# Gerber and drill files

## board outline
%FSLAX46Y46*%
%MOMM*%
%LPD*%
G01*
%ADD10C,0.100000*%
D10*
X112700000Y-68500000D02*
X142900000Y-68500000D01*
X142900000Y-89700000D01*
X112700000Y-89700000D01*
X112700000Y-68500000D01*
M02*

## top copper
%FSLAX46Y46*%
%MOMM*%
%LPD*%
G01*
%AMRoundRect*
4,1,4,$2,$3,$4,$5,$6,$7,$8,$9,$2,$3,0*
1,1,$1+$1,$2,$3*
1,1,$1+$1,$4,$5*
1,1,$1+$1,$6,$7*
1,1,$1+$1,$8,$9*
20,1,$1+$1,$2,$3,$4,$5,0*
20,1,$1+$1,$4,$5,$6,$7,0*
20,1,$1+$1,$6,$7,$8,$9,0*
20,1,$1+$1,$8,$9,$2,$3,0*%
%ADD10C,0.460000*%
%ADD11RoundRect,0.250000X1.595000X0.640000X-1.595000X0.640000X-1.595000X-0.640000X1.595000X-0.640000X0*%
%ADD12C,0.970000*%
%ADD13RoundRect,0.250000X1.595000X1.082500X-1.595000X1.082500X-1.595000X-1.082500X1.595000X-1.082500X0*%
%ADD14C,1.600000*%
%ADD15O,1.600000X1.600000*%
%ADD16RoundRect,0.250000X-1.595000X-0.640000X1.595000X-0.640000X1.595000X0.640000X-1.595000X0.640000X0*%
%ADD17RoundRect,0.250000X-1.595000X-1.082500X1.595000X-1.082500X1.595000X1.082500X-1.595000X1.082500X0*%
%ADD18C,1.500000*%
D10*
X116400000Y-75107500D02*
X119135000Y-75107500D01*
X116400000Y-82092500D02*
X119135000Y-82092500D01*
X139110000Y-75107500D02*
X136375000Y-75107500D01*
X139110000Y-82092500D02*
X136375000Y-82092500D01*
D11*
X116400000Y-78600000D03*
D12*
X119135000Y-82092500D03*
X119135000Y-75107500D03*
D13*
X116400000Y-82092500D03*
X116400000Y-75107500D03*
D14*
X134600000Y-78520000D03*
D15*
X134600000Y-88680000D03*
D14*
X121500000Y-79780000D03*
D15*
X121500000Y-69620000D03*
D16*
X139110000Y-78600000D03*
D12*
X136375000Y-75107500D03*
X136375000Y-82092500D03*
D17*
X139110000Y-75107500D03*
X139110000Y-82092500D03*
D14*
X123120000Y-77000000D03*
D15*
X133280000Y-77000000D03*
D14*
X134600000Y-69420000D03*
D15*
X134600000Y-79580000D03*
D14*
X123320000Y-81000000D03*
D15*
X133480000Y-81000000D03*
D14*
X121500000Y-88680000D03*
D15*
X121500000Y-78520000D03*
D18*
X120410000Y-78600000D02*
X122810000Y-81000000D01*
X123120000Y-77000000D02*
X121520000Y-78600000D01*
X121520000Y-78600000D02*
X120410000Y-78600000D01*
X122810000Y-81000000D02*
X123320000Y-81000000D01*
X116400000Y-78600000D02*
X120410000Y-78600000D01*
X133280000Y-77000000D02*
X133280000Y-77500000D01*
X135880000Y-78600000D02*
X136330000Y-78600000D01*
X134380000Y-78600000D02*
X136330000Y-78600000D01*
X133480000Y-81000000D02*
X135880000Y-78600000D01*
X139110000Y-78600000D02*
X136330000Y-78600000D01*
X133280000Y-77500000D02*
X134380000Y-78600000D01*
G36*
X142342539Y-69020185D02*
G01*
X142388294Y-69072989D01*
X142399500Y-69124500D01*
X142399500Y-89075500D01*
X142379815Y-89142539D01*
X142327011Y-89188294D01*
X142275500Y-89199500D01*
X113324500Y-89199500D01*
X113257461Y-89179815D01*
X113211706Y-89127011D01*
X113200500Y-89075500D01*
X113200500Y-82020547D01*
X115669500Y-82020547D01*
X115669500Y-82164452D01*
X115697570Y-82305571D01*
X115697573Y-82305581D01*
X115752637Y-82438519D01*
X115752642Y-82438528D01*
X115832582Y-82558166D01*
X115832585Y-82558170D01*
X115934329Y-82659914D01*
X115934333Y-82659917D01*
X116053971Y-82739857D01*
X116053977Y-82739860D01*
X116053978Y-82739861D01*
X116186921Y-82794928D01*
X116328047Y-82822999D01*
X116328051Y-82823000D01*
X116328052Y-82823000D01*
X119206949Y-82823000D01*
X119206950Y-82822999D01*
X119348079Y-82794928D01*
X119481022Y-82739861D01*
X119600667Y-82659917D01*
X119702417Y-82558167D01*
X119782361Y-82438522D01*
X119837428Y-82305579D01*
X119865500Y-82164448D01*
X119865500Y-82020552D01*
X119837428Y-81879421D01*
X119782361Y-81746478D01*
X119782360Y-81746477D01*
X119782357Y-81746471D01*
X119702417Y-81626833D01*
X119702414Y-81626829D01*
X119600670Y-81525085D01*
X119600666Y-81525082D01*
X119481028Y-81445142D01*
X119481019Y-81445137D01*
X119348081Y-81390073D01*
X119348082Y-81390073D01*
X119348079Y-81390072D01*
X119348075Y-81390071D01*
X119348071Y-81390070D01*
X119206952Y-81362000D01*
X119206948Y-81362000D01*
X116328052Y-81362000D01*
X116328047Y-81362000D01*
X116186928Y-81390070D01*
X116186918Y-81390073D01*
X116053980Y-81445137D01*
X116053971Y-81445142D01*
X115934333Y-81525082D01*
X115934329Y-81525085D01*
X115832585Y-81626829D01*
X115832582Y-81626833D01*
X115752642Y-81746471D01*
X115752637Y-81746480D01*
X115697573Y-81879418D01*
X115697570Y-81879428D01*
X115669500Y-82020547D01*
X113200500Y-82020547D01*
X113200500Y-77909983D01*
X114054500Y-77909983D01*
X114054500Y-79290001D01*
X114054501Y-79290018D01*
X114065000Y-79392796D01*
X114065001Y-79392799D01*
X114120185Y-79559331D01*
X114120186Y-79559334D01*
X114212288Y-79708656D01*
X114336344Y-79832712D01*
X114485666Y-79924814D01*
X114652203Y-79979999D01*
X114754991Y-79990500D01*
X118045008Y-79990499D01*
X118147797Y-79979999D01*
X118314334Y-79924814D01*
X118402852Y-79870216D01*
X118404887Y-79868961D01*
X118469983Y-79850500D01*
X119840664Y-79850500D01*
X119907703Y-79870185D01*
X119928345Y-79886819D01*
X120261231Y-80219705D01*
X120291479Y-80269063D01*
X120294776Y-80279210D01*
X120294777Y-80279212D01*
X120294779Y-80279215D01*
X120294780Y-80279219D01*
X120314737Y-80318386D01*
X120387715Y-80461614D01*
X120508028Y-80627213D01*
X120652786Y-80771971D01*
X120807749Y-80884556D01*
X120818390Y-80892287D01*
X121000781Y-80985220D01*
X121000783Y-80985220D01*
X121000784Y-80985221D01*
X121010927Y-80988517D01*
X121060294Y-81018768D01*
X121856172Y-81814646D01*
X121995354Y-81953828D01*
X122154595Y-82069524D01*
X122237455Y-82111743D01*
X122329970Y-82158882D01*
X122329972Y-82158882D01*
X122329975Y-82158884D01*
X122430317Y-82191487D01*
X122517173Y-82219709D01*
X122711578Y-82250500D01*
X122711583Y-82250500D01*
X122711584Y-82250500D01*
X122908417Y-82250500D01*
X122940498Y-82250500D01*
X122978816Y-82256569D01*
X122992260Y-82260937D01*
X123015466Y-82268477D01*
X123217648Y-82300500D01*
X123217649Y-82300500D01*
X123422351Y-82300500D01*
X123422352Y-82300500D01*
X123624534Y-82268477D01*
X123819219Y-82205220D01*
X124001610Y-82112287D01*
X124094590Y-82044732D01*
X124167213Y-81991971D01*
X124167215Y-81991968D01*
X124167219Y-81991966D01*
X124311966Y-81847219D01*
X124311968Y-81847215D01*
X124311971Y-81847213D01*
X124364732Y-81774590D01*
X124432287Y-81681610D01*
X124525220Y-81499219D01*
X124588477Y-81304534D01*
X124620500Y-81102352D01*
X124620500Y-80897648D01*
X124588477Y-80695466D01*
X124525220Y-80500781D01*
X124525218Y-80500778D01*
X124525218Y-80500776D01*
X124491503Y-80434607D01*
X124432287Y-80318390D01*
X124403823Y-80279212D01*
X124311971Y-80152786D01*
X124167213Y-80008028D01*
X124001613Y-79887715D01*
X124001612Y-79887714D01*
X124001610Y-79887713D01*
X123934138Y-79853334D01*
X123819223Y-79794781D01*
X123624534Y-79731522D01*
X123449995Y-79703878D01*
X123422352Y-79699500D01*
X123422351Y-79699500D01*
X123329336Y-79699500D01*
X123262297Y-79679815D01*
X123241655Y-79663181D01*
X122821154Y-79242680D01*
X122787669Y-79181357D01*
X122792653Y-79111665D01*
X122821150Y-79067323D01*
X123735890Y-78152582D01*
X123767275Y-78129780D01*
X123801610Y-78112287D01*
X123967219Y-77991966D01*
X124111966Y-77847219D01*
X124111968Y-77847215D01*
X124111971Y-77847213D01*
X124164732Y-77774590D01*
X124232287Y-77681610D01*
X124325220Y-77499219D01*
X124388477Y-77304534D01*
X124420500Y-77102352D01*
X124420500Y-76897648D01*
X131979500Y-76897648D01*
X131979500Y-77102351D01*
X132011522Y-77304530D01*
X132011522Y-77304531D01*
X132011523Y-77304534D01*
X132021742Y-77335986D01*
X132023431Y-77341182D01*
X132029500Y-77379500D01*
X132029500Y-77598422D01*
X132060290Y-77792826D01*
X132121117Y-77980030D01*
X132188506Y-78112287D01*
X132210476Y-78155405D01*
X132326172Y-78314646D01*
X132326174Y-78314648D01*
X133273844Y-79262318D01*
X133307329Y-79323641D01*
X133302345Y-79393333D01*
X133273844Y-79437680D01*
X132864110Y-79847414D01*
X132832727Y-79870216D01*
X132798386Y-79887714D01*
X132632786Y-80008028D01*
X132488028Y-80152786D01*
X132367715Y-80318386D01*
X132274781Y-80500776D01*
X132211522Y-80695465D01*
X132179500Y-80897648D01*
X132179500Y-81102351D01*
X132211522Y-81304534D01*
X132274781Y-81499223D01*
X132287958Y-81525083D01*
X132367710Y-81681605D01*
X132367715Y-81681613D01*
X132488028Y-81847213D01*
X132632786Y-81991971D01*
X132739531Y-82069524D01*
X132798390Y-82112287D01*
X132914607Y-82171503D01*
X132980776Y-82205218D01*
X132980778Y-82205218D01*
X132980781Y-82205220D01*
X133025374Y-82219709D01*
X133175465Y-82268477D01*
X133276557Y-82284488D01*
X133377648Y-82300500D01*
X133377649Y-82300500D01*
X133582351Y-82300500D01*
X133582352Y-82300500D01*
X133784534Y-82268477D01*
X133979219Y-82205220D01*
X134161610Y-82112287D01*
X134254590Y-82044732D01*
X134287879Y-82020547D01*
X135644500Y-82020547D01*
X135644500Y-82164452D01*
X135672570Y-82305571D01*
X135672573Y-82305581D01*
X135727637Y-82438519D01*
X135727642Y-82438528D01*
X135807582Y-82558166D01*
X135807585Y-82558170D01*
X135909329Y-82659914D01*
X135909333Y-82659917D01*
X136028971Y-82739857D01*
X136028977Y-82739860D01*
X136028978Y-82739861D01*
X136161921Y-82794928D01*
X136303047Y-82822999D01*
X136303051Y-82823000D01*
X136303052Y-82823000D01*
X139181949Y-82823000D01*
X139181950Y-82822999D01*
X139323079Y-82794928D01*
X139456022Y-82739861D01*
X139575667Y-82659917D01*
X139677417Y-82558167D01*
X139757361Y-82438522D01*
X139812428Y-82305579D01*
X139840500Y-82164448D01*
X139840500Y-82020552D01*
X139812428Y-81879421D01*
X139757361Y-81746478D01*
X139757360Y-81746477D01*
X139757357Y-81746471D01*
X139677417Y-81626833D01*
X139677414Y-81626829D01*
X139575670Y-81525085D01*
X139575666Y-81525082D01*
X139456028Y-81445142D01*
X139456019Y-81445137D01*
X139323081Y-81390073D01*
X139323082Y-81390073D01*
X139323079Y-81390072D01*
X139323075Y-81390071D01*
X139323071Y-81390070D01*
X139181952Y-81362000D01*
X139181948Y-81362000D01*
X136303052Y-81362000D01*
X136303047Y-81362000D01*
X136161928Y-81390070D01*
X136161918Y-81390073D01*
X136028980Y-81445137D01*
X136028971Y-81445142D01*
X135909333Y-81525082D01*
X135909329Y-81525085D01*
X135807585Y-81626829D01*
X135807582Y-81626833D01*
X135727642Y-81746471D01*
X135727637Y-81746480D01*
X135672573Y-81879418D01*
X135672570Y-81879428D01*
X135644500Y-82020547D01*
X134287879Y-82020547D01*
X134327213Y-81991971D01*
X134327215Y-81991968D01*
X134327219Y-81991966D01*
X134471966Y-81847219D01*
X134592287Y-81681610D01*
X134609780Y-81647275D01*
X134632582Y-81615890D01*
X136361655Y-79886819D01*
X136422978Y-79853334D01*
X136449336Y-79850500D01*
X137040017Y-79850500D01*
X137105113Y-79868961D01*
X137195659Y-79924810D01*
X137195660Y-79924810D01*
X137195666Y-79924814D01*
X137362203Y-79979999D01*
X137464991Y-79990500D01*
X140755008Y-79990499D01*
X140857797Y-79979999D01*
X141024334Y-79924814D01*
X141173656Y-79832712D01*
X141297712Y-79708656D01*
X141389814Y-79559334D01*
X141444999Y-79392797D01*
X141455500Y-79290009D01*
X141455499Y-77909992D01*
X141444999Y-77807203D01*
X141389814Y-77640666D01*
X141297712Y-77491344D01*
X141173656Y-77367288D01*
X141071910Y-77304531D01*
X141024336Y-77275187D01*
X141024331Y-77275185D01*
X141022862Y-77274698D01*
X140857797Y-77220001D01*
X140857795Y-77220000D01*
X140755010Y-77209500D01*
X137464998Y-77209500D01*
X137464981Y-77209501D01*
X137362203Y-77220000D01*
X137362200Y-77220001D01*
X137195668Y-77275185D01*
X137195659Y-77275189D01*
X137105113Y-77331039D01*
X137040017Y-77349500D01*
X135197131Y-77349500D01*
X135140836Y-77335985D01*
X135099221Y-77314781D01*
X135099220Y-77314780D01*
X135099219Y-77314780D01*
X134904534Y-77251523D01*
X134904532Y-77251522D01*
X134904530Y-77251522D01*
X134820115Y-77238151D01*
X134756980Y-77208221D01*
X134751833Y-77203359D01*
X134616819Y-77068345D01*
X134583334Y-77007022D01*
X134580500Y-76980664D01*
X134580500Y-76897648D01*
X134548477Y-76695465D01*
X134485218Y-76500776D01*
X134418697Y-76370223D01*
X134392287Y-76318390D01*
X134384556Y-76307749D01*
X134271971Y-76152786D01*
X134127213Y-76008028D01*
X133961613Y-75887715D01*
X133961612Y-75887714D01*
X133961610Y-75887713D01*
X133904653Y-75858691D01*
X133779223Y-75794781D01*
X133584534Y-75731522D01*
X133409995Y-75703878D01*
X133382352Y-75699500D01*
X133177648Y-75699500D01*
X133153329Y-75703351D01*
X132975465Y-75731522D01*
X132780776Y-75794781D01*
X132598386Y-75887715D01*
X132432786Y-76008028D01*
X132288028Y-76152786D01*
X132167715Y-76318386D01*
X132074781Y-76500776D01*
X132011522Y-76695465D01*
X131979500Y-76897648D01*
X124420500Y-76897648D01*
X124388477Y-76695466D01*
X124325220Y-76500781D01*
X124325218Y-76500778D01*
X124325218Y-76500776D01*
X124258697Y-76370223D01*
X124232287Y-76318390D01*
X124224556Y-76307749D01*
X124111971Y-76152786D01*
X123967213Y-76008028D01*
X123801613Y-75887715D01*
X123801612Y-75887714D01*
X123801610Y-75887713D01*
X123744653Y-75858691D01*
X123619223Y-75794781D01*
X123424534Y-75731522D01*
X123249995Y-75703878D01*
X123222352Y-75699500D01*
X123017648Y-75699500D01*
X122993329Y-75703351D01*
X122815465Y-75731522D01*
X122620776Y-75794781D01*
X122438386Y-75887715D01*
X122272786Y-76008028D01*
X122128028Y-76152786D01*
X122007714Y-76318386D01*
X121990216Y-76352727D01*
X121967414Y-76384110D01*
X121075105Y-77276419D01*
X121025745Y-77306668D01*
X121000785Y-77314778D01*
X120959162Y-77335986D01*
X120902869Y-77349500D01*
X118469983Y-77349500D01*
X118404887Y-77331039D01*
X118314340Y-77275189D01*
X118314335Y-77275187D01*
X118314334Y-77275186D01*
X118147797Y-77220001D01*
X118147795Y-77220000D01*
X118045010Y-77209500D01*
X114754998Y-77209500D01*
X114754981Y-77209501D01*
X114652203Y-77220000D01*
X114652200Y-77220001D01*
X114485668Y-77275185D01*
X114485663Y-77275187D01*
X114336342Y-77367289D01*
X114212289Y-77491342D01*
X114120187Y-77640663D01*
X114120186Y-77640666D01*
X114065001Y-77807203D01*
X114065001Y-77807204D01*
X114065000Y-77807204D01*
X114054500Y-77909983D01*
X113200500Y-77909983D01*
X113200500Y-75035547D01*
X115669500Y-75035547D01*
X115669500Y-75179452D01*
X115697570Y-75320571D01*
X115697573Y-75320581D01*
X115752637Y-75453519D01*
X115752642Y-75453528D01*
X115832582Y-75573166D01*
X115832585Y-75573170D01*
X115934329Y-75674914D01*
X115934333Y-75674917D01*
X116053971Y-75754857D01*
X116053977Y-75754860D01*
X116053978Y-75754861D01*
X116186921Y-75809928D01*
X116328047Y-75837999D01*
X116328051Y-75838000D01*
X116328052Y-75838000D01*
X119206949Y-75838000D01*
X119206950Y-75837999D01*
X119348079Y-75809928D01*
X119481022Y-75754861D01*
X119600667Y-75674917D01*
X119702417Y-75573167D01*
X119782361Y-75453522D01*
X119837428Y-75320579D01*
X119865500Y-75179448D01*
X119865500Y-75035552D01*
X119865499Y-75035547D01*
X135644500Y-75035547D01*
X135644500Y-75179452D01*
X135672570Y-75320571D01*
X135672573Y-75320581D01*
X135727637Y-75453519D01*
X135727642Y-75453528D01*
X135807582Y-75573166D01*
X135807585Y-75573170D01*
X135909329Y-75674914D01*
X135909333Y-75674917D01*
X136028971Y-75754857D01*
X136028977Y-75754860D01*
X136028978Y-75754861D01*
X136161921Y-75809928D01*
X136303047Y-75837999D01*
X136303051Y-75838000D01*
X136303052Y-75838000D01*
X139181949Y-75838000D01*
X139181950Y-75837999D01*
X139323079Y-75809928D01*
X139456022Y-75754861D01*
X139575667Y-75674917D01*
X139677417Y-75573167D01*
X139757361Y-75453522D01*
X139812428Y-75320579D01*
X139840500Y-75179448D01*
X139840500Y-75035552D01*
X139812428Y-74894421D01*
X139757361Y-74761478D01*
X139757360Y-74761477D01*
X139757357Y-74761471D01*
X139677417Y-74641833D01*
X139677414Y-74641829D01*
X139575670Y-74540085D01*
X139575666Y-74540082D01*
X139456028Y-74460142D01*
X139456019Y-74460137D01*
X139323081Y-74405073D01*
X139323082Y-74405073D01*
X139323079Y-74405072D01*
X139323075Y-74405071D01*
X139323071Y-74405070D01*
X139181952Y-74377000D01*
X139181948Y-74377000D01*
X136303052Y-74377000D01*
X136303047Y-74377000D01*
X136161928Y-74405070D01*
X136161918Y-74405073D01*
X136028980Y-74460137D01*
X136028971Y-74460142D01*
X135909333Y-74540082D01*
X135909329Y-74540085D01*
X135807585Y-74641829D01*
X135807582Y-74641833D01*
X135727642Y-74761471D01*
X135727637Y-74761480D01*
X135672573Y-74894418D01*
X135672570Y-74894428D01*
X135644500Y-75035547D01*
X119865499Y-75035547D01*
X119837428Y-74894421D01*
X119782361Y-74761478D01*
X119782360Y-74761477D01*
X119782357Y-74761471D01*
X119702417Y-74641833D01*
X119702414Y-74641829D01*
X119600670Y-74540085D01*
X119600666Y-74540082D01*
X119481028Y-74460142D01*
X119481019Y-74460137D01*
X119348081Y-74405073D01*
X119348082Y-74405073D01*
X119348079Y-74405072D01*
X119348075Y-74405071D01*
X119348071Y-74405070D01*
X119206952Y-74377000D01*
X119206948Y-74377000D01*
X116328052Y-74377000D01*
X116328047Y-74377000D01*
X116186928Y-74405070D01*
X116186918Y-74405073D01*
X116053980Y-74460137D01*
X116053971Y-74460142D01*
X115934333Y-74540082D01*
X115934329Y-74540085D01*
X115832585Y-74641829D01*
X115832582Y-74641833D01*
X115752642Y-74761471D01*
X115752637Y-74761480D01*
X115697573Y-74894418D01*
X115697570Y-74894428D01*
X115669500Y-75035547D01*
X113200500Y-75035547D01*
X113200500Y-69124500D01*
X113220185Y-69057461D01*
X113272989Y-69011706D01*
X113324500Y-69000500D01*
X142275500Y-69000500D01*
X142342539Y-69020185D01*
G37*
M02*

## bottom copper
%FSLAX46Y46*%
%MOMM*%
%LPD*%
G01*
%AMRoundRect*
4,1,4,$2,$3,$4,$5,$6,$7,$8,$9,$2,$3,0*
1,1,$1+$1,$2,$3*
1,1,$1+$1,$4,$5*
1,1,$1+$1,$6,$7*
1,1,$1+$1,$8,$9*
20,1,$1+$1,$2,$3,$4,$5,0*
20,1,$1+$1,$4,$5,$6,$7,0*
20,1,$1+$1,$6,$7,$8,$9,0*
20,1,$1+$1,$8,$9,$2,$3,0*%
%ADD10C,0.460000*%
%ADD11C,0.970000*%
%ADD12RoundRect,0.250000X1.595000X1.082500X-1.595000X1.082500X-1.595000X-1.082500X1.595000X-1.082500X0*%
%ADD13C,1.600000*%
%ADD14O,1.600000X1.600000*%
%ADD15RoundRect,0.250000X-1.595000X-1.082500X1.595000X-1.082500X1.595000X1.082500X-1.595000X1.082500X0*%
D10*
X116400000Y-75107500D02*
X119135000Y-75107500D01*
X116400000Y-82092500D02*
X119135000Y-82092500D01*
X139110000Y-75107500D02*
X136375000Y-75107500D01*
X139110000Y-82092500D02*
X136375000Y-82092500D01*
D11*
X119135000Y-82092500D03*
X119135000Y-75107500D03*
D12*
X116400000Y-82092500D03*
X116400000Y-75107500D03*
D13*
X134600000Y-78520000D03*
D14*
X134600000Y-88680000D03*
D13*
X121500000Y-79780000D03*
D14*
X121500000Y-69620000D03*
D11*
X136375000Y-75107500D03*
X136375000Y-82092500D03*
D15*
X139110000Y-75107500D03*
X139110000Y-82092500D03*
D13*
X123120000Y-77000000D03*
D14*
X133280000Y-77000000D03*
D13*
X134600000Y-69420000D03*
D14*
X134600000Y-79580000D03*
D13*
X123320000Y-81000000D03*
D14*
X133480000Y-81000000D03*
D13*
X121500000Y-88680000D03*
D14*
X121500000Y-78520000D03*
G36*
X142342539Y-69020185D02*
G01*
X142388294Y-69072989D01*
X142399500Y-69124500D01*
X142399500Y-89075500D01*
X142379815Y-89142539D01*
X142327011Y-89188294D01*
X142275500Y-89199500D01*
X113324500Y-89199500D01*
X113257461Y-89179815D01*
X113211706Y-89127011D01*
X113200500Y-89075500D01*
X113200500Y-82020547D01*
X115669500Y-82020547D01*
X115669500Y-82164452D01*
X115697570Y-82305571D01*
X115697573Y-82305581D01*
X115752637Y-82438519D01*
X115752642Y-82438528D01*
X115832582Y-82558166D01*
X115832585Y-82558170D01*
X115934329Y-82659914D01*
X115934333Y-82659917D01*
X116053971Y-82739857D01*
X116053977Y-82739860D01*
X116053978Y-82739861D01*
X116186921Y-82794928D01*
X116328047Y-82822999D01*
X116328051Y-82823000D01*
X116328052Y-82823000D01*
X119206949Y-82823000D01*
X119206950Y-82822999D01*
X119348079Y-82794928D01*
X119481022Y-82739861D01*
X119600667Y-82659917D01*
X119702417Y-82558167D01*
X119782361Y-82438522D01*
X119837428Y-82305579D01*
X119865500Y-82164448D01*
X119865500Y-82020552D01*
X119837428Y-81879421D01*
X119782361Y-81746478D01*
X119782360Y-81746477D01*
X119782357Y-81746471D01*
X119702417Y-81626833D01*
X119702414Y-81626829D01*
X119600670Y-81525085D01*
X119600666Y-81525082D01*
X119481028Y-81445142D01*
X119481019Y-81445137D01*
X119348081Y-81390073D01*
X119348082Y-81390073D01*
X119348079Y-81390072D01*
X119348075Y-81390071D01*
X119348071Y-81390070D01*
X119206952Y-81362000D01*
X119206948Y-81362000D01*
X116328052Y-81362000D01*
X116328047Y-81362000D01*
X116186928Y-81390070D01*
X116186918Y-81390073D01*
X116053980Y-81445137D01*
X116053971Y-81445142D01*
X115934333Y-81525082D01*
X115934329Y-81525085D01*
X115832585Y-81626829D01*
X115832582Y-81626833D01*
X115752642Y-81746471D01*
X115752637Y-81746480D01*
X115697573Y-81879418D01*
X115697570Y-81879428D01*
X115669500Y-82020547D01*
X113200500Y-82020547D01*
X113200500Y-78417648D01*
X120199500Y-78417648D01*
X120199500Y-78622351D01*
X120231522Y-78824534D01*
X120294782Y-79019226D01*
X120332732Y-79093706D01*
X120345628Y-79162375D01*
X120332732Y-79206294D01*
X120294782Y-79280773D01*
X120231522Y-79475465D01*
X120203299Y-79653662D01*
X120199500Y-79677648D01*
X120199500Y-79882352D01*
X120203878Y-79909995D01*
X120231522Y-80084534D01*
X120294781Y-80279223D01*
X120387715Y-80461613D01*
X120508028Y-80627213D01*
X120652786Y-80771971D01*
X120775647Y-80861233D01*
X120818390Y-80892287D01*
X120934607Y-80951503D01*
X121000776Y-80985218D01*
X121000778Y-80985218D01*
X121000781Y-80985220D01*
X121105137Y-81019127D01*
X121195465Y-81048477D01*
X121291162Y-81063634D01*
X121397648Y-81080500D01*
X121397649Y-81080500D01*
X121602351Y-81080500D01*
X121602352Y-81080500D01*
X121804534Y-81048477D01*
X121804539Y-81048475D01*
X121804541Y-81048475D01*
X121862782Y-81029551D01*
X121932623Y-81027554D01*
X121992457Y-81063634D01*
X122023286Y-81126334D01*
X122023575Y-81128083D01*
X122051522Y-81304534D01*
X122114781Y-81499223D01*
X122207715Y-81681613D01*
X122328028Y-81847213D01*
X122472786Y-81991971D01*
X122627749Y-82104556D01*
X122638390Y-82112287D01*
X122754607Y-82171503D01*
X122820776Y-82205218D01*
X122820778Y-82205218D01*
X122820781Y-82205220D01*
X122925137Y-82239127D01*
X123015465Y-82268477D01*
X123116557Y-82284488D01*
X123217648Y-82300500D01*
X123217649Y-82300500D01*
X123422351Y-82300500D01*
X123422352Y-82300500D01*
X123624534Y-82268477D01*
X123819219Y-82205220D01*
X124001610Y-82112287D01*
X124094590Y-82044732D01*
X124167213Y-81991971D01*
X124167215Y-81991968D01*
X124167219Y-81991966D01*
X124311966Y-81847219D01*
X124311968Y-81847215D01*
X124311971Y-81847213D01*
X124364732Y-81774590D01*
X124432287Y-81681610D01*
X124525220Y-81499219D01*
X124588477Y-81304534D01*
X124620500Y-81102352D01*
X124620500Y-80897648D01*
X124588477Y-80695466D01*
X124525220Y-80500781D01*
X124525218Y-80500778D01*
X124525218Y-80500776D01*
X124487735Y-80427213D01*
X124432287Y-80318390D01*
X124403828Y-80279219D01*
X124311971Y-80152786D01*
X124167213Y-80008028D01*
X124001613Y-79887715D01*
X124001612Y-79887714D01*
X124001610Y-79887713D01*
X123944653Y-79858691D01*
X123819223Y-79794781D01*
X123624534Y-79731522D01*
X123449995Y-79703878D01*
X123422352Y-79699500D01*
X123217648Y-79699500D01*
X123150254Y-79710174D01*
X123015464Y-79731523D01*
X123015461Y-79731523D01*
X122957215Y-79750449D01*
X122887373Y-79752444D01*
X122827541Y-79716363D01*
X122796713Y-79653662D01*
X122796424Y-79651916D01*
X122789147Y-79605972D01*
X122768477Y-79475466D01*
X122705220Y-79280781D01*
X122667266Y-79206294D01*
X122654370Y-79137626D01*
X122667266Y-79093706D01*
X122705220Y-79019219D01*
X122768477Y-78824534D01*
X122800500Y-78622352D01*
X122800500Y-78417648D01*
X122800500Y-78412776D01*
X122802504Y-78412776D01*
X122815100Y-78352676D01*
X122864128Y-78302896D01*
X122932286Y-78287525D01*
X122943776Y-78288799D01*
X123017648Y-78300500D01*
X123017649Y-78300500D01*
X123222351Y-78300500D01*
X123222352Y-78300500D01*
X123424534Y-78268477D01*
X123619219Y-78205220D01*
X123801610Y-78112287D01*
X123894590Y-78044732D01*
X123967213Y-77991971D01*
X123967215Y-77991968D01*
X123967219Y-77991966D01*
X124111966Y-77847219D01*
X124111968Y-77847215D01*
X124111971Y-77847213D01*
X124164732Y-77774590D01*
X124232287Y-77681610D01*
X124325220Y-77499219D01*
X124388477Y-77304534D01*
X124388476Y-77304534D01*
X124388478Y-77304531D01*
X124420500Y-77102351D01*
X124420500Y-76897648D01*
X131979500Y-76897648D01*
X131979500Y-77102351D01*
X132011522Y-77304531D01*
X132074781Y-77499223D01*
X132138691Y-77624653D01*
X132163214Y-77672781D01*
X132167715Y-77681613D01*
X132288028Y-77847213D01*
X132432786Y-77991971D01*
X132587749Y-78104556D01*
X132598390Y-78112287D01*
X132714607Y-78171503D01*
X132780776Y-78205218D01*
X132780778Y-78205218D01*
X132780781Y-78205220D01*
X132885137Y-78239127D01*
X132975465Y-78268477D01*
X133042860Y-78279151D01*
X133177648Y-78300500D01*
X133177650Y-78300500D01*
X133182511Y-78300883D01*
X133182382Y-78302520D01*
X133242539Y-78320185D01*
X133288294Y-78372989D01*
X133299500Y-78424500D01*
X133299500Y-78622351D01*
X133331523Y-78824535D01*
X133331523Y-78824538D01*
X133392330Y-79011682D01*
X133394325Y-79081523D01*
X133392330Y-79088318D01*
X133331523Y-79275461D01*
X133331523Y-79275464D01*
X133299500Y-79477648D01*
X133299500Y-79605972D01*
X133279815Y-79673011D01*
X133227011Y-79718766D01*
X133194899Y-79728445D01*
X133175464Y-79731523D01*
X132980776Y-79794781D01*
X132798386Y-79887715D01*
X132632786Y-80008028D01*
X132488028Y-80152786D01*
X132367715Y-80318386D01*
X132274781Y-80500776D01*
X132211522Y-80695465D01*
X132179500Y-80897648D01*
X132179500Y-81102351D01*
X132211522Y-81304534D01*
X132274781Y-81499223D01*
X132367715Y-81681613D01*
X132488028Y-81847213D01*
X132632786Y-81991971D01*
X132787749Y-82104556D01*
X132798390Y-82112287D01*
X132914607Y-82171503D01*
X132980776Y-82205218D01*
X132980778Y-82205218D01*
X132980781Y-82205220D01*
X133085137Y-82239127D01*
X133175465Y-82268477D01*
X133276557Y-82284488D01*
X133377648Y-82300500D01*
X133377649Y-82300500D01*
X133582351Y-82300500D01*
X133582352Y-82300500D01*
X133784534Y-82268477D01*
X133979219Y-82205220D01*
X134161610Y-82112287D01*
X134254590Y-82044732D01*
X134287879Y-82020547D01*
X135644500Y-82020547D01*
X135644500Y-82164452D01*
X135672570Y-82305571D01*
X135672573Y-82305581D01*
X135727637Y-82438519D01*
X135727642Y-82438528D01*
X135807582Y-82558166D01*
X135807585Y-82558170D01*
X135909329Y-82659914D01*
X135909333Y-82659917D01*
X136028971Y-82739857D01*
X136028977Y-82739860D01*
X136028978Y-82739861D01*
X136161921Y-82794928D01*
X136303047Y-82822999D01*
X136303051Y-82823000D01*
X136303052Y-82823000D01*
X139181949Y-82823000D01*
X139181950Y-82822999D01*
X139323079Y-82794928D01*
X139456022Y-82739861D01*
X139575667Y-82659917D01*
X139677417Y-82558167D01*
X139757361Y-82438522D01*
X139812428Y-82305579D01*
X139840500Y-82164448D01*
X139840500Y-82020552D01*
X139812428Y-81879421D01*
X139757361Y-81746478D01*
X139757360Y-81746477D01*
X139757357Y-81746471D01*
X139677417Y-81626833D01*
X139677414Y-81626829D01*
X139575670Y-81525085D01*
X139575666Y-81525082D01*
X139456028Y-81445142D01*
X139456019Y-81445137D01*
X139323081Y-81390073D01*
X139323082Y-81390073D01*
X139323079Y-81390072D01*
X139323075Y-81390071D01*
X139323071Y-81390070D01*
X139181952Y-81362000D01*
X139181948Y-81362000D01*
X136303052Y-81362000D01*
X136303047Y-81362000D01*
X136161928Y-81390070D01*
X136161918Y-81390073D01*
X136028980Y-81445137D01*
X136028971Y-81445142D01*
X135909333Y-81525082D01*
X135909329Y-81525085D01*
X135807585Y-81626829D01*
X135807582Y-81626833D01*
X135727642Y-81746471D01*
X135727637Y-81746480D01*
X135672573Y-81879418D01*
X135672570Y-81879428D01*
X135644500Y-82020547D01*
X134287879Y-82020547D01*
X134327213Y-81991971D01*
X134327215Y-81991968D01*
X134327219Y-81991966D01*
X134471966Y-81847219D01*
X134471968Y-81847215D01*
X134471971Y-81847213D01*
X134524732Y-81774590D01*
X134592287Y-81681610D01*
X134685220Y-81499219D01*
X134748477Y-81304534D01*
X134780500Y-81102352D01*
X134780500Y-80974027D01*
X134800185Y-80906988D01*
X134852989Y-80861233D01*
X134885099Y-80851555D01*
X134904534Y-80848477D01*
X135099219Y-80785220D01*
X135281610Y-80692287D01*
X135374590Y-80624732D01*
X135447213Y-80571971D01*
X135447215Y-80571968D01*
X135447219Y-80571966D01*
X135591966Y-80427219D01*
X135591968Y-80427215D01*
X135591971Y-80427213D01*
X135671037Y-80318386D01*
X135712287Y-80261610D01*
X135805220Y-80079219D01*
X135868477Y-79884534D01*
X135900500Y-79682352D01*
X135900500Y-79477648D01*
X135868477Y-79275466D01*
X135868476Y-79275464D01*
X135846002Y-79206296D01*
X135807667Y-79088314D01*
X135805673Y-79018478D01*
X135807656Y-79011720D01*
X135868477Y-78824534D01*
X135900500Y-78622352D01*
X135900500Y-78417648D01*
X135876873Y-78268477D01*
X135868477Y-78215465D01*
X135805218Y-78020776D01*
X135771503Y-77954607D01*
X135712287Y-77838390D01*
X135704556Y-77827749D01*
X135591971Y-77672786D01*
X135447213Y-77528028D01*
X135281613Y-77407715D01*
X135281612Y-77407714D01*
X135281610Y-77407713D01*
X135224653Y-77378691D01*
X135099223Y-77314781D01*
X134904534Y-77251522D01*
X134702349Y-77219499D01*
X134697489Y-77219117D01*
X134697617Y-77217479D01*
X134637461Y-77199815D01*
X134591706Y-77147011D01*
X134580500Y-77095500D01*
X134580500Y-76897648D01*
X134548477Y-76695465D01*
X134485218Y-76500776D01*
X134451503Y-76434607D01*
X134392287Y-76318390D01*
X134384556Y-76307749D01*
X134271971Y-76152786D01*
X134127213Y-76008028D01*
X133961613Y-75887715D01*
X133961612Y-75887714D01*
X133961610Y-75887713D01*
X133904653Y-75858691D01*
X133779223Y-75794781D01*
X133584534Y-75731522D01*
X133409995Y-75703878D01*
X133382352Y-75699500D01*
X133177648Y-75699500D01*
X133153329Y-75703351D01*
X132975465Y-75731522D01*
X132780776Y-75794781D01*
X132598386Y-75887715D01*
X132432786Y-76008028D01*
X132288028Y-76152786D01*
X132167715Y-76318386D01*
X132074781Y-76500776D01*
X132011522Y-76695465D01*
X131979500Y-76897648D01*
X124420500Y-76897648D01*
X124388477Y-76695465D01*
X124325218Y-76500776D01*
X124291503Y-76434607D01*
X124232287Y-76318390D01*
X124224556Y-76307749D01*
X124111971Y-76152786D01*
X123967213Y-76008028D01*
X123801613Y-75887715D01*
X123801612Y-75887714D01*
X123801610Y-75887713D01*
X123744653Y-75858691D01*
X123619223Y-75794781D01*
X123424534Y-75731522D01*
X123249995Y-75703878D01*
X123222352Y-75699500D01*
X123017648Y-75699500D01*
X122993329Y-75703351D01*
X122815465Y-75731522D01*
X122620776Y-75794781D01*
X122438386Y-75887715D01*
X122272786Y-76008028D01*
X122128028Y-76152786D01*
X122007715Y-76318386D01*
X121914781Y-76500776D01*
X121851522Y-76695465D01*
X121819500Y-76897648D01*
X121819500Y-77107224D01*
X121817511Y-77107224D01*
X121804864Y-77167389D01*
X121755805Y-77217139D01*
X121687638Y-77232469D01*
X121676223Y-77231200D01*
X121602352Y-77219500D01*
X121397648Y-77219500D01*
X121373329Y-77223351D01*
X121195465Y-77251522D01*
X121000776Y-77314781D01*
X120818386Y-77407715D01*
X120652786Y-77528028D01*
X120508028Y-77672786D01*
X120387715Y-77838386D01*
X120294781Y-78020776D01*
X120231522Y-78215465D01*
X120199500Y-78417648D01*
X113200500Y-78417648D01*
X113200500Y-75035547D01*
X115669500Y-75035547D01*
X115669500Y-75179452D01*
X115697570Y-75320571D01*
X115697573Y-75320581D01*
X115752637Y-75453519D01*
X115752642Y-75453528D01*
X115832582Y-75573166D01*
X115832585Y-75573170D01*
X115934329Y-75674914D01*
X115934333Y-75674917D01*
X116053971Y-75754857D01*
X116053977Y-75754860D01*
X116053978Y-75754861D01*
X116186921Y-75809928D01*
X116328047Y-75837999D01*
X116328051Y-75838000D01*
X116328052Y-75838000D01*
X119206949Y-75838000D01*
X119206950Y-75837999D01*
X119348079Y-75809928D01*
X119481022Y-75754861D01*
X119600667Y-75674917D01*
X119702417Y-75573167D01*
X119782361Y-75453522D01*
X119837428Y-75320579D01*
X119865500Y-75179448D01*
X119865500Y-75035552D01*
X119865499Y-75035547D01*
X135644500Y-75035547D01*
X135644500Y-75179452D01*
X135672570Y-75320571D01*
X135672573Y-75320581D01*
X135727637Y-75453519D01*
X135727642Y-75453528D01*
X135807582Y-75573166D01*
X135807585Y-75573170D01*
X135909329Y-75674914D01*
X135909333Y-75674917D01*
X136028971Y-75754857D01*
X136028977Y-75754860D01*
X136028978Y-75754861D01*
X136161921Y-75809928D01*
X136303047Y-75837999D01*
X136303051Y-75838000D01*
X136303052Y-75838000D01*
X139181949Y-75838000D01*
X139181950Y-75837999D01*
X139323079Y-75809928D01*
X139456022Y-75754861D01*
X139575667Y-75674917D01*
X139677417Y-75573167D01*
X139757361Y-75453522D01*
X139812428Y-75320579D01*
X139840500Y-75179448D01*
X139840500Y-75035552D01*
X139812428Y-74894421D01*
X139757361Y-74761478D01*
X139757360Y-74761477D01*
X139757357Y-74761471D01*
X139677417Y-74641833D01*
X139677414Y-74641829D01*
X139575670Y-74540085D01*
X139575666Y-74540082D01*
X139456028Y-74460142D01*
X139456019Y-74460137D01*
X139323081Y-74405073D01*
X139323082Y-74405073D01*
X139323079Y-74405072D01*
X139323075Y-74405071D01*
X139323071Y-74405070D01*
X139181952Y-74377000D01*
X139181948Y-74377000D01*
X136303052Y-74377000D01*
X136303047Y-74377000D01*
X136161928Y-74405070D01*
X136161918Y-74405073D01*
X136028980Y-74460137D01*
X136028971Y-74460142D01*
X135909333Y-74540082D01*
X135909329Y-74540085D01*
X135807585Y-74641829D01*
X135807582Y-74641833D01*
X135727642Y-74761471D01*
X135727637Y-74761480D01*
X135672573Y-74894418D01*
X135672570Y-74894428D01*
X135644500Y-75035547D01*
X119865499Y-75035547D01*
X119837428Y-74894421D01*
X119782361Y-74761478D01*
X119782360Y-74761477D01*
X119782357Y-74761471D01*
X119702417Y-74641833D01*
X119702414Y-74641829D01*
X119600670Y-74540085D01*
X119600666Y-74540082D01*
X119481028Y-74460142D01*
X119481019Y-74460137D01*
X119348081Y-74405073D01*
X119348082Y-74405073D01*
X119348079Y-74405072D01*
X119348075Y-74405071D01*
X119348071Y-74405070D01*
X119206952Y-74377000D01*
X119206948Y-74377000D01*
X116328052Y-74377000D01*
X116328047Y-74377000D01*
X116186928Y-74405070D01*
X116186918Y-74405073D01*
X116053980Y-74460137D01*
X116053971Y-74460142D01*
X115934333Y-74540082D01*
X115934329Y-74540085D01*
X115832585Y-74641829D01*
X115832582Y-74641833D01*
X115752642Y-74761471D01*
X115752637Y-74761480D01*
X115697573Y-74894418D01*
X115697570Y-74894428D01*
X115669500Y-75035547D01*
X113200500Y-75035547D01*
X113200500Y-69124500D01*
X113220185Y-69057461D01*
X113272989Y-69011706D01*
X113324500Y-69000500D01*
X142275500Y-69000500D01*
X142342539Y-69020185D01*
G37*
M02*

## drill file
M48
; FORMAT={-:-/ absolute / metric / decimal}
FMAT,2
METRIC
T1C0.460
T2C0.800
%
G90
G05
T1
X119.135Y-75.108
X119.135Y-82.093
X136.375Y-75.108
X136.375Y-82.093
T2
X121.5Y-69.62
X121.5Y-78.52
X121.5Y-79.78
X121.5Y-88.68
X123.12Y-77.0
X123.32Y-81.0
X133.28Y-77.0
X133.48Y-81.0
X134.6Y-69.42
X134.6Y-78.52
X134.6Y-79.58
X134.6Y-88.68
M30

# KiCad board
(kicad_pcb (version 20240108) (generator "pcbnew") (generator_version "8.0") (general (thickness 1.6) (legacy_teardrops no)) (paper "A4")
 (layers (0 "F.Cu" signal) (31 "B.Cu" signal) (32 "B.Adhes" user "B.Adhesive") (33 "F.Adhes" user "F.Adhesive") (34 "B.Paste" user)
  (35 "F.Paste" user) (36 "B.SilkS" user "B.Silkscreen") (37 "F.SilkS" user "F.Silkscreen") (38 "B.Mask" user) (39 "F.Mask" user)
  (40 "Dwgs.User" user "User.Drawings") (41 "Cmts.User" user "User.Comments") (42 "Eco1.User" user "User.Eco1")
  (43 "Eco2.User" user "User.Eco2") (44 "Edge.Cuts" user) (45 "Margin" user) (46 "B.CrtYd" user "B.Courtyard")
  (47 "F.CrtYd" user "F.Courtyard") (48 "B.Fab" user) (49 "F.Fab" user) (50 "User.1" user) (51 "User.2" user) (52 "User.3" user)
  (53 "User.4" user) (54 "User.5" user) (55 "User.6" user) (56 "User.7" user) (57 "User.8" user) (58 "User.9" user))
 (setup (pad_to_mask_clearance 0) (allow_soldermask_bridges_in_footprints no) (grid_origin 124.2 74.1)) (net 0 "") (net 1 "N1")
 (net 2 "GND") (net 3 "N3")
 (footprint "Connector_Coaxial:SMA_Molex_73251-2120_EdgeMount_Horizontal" (layer "F.Cu") (at 116.15 78.6 180)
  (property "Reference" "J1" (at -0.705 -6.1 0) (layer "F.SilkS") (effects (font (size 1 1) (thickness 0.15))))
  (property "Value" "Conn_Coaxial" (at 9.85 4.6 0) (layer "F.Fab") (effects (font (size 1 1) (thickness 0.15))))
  (fp_line (start -0.25 3.4925) (end -2.985 3.4925) (stroke (width 0.46) (type default)) (layer "F.Cu"))
  (fp_line (start -0.25 -3.4925) (end -2.985 -3.4925) (stroke (width 0.46) (type default)) (layer "F.Cu"))
  (fp_line (start -0.25 3.4925) (end -2.985 3.4925) (stroke (width 0.46) (type default)) (layer "B.Cu"))
  (fp_line (start -0.25 -3.4925) (end -2.985 -3.4925) (stroke (width 0.46) (type default)) (layer "B.Cu"))
  (pad "1" smd roundrect (at -0.25 0 180) (size 3.69 1.78) (layers "F.Cu" "F.Paste" "F.Mask") (roundrect_rratio 0.1404494382) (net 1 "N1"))
  (pad "2" thru_hole circle (at -2.985 -3.4925 180) (size 0.97 0.97) (drill 0.46) (layers "*.Cu") (remove_unused_layers no) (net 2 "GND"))
  (pad "2" thru_hole circle (at -2.985 3.4925 180) (size 0.97 0.97) (drill 0.46) (layers "*.Cu") (remove_unused_layers no) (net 2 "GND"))
  (pad "2" smd roundrect (at -0.25 -3.4925 180) (size 3.69 2.665) (layers "F.Cu" "F.Paste" "F.Mask") (roundrect_rratio 0.09380863039)
   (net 2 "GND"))
  (pad "2" smd roundrect (at -0.25 -3.4925 180) (size 3.69 2.665) (layers "B.Cu" "B.Paste" "B.Mask") (roundrect_rratio 0.09380863039)
   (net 2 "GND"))
  (pad "2" smd roundrect (at -0.25 3.4925 180) (size 3.69 2.665) (layers "F.Cu" "F.Paste" "F.Mask") (roundrect_rratio 0.09380863039)
   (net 2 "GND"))
  (pad "2" smd roundrect (at -0.25 3.4925 180) (size 3.69 2.665) (layers "B.Cu" "B.Paste" "B.Mask") (roundrect_rratio 0.09380863039)
   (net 2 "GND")))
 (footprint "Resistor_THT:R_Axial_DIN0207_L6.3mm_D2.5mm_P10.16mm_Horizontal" (layer "F.Cu") (at 134.6 78.52 -90)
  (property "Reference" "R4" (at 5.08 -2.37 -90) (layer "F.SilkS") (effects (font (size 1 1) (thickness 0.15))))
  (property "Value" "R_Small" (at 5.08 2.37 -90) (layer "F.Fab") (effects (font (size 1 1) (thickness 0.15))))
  (pad "1" thru_hole circle (at 0 0 270) (size 1.6 1.6) (drill 0.8) (layers "*.Cu" "*.Mask") (remove_unused_layers no) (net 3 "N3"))
  (pad "2" thru_hole oval (at 10.16 0 270) (size 1.6 1.6) (drill 0.8) (layers "*.Cu" "*.Mask") (remove_unused_layers no) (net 2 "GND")))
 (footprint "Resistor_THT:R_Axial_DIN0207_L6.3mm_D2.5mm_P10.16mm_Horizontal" (layer "F.Cu") (at 121.5 79.78 90)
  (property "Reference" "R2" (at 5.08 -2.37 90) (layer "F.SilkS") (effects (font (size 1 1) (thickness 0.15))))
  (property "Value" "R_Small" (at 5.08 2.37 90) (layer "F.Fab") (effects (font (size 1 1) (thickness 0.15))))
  (pad "1" thru_hole circle (at 0 0 90) (size 1.6 1.6) (drill 0.8) (layers "*.Cu" "*.Mask") (remove_unused_layers no) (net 1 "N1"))
  (pad "2" thru_hole oval (at 10.16 0 90) (size 1.6 1.6) (drill 0.8) (layers "*.Cu" "*.Mask") (remove_unused_layers no) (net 2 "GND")))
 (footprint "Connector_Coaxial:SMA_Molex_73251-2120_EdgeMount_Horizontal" (layer "F.Cu") (at 139.36 78.6)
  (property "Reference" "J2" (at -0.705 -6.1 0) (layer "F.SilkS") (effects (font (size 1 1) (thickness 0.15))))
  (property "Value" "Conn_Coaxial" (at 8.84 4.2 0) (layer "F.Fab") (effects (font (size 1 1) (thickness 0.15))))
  (fp_line (start -0.25 -3.4925) (end -2.985 -3.4925) (stroke (width 0.46) (type default)) (layer "F.Cu"))
  (fp_line (start -0.25 3.4925) (end -2.985 3.4925) (stroke (width 0.46) (type default)) (layer "F.Cu"))
  (fp_line (start -0.25 -3.4925) (end -2.985 -3.4925) (stroke (width 0.46) (type default)) (layer "B.Cu"))
  (fp_line (start -0.25 3.4925) (end -2.985 3.4925) (stroke (width 0.46) (type default)) (layer "B.Cu"))
  (pad "1" smd roundrect (at -0.25 0) (size 3.69 1.78) (layers "F.Cu" "F.Paste" "F.Mask") (roundrect_rratio 0.1404494382) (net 3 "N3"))
  (pad "2" thru_hole circle (at -2.985 -3.4925) (size 0.97 0.97) (drill 0.46) (layers "*.Cu") (remove_unused_layers no) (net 2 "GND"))
  (pad "2" thru_hole circle (at -2.985 3.4925) (size 0.97 0.97) (drill 0.46) (layers "*.Cu") (remove_unused_layers no) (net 2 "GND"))
  (pad "2" smd roundrect (at -0.25 -3.4925) (size 3.69 2.665) (layers "F.Cu" "F.Paste" "F.Mask") (roundrect_rratio 0.09380863039)
   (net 2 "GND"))
  (pad "2" smd roundrect (at -0.25 -3.4925) (size 3.69 2.665) (layers "B.Cu" "B.Paste" "B.Mask") (roundrect_rratio 0.09380863039)
   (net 2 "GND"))
  (pad "2" smd roundrect (at -0.25 3.4925) (size 3.69 2.665) (layers "F.Cu" "F.Paste" "F.Mask") (roundrect_rratio 0.09380863039)
   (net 2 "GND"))
  (pad "2" smd roundrect (at -0.25 3.4925) (size 3.69 2.665) (layers "B.Cu" "B.Paste" "B.Mask") (roundrect_rratio 0.09380863039)
   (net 2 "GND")))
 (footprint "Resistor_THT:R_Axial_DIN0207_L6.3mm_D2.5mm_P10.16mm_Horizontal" (layer "F.Cu") (at 123.12 77)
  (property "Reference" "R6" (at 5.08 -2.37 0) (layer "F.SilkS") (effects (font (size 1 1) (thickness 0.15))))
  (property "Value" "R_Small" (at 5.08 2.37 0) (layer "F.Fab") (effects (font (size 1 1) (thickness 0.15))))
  (pad "1" thru_hole circle (at 0 0) (size 1.6 1.6) (drill 0.8) (layers "*.Cu" "*.Mask") (remove_unused_layers no) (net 1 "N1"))
  (pad "2" thru_hole oval (at 10.16 0) (size 1.6 1.6) (drill 0.8) (layers "*.Cu" "*.Mask") (remove_unused_layers no) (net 3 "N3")))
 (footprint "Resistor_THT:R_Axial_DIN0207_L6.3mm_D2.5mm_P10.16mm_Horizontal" (layer "F.Cu") (at 134.6 69.42 -90)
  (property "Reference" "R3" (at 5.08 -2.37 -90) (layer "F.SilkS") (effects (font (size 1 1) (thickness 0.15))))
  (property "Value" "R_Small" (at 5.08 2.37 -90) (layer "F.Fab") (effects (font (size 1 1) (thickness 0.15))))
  (pad "1" thru_hole circle (at 0 0 270) (size 1.6 1.6) (drill 0.8) (layers "*.Cu" "*.Mask") (remove_unused_layers no) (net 2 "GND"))
  (pad "2" thru_hole oval (at 10.16 0 270) (size 1.6 1.6) (drill 0.8) (layers "*.Cu" "*.Mask") (remove_unused_layers no) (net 3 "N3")))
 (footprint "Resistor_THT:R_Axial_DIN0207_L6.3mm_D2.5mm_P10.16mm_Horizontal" (layer "F.Cu") (at 123.32 81)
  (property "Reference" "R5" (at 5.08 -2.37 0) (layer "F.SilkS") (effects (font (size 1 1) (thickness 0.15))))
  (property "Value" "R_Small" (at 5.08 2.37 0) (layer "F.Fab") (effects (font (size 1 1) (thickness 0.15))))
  (pad "1" thru_hole circle (at 0 0) (size 1.6 1.6) (drill 0.8) (layers "*.Cu" "*.Mask") (remove_unused_layers no) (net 1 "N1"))
  (pad "2" thru_hole oval (at 10.16 0) (size 1.6 1.6) (drill 0.8) (layers "*.Cu" "*.Mask") (remove_unused_layers no) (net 3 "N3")))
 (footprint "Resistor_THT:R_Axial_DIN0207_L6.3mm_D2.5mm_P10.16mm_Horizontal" (layer "F.Cu") (at 121.5 88.68 90)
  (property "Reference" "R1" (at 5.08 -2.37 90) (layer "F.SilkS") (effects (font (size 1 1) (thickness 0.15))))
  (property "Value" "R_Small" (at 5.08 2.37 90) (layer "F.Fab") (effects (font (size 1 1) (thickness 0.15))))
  (pad "1" thru_hole circle (at 0 0 90) (size 1.6 1.6) (drill 0.8) (layers "*.Cu" "*.Mask") (remove_unused_layers no) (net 2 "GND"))
  (pad "2" thru_hole oval (at 10.16 0 90) (size 1.6 1.6) (drill 0.8) (layers "*.Cu" "*.Mask") (remove_unused_layers no) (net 1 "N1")))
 (gr_rect (start 112.7 68.5) (end 142.9 89.7) (stroke (width 0.1) (type default)) (fill none) (layer "Edge.Cuts"))
 (segment (start 120.41 78.6) (end 122.81 81) (width 1.5) (layer "F.Cu") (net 1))
 (segment (start 123.12 77) (end 121.52 78.6) (width 1.5) (layer "F.Cu") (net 1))
 (segment (start 121.52 78.6) (end 120.41 78.6) (width 1.5) (layer "F.Cu") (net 1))
 (segment (start 122.81 81) (end 123.32 81) (width 1.5) (layer "F.Cu") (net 1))
 (segment (start 116.4 78.6) (end 120.41 78.6) (width 1.5) (layer "F.Cu") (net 1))
 (segment (start 133.28 77) (end 133.28 77.5) (width 1.5) (layer "F.Cu") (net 3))
 (segment (start 135.88 78.6) (end 136.33 78.6) (width 1.5) (layer "F.Cu") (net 3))
 (segment (start 134.38 78.6) (end 136.33 78.6) (width 1.5) (layer "F.Cu") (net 3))
 (segment (start 133.48 81) (end 135.88 78.6) (width 1.5) (layer "F.Cu") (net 3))
 (segment (start 139.11 78.6) (end 136.33 78.6) (width 1.5) (layer "F.Cu") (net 3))
 (segment (start 133.28 77.5) (end 134.38 78.6) (width 1.5) (layer "F.Cu") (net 3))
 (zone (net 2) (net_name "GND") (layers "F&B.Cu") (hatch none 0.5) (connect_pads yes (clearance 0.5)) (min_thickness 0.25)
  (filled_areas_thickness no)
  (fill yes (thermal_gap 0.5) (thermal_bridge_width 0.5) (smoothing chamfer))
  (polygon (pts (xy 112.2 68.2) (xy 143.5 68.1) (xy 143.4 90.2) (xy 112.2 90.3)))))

